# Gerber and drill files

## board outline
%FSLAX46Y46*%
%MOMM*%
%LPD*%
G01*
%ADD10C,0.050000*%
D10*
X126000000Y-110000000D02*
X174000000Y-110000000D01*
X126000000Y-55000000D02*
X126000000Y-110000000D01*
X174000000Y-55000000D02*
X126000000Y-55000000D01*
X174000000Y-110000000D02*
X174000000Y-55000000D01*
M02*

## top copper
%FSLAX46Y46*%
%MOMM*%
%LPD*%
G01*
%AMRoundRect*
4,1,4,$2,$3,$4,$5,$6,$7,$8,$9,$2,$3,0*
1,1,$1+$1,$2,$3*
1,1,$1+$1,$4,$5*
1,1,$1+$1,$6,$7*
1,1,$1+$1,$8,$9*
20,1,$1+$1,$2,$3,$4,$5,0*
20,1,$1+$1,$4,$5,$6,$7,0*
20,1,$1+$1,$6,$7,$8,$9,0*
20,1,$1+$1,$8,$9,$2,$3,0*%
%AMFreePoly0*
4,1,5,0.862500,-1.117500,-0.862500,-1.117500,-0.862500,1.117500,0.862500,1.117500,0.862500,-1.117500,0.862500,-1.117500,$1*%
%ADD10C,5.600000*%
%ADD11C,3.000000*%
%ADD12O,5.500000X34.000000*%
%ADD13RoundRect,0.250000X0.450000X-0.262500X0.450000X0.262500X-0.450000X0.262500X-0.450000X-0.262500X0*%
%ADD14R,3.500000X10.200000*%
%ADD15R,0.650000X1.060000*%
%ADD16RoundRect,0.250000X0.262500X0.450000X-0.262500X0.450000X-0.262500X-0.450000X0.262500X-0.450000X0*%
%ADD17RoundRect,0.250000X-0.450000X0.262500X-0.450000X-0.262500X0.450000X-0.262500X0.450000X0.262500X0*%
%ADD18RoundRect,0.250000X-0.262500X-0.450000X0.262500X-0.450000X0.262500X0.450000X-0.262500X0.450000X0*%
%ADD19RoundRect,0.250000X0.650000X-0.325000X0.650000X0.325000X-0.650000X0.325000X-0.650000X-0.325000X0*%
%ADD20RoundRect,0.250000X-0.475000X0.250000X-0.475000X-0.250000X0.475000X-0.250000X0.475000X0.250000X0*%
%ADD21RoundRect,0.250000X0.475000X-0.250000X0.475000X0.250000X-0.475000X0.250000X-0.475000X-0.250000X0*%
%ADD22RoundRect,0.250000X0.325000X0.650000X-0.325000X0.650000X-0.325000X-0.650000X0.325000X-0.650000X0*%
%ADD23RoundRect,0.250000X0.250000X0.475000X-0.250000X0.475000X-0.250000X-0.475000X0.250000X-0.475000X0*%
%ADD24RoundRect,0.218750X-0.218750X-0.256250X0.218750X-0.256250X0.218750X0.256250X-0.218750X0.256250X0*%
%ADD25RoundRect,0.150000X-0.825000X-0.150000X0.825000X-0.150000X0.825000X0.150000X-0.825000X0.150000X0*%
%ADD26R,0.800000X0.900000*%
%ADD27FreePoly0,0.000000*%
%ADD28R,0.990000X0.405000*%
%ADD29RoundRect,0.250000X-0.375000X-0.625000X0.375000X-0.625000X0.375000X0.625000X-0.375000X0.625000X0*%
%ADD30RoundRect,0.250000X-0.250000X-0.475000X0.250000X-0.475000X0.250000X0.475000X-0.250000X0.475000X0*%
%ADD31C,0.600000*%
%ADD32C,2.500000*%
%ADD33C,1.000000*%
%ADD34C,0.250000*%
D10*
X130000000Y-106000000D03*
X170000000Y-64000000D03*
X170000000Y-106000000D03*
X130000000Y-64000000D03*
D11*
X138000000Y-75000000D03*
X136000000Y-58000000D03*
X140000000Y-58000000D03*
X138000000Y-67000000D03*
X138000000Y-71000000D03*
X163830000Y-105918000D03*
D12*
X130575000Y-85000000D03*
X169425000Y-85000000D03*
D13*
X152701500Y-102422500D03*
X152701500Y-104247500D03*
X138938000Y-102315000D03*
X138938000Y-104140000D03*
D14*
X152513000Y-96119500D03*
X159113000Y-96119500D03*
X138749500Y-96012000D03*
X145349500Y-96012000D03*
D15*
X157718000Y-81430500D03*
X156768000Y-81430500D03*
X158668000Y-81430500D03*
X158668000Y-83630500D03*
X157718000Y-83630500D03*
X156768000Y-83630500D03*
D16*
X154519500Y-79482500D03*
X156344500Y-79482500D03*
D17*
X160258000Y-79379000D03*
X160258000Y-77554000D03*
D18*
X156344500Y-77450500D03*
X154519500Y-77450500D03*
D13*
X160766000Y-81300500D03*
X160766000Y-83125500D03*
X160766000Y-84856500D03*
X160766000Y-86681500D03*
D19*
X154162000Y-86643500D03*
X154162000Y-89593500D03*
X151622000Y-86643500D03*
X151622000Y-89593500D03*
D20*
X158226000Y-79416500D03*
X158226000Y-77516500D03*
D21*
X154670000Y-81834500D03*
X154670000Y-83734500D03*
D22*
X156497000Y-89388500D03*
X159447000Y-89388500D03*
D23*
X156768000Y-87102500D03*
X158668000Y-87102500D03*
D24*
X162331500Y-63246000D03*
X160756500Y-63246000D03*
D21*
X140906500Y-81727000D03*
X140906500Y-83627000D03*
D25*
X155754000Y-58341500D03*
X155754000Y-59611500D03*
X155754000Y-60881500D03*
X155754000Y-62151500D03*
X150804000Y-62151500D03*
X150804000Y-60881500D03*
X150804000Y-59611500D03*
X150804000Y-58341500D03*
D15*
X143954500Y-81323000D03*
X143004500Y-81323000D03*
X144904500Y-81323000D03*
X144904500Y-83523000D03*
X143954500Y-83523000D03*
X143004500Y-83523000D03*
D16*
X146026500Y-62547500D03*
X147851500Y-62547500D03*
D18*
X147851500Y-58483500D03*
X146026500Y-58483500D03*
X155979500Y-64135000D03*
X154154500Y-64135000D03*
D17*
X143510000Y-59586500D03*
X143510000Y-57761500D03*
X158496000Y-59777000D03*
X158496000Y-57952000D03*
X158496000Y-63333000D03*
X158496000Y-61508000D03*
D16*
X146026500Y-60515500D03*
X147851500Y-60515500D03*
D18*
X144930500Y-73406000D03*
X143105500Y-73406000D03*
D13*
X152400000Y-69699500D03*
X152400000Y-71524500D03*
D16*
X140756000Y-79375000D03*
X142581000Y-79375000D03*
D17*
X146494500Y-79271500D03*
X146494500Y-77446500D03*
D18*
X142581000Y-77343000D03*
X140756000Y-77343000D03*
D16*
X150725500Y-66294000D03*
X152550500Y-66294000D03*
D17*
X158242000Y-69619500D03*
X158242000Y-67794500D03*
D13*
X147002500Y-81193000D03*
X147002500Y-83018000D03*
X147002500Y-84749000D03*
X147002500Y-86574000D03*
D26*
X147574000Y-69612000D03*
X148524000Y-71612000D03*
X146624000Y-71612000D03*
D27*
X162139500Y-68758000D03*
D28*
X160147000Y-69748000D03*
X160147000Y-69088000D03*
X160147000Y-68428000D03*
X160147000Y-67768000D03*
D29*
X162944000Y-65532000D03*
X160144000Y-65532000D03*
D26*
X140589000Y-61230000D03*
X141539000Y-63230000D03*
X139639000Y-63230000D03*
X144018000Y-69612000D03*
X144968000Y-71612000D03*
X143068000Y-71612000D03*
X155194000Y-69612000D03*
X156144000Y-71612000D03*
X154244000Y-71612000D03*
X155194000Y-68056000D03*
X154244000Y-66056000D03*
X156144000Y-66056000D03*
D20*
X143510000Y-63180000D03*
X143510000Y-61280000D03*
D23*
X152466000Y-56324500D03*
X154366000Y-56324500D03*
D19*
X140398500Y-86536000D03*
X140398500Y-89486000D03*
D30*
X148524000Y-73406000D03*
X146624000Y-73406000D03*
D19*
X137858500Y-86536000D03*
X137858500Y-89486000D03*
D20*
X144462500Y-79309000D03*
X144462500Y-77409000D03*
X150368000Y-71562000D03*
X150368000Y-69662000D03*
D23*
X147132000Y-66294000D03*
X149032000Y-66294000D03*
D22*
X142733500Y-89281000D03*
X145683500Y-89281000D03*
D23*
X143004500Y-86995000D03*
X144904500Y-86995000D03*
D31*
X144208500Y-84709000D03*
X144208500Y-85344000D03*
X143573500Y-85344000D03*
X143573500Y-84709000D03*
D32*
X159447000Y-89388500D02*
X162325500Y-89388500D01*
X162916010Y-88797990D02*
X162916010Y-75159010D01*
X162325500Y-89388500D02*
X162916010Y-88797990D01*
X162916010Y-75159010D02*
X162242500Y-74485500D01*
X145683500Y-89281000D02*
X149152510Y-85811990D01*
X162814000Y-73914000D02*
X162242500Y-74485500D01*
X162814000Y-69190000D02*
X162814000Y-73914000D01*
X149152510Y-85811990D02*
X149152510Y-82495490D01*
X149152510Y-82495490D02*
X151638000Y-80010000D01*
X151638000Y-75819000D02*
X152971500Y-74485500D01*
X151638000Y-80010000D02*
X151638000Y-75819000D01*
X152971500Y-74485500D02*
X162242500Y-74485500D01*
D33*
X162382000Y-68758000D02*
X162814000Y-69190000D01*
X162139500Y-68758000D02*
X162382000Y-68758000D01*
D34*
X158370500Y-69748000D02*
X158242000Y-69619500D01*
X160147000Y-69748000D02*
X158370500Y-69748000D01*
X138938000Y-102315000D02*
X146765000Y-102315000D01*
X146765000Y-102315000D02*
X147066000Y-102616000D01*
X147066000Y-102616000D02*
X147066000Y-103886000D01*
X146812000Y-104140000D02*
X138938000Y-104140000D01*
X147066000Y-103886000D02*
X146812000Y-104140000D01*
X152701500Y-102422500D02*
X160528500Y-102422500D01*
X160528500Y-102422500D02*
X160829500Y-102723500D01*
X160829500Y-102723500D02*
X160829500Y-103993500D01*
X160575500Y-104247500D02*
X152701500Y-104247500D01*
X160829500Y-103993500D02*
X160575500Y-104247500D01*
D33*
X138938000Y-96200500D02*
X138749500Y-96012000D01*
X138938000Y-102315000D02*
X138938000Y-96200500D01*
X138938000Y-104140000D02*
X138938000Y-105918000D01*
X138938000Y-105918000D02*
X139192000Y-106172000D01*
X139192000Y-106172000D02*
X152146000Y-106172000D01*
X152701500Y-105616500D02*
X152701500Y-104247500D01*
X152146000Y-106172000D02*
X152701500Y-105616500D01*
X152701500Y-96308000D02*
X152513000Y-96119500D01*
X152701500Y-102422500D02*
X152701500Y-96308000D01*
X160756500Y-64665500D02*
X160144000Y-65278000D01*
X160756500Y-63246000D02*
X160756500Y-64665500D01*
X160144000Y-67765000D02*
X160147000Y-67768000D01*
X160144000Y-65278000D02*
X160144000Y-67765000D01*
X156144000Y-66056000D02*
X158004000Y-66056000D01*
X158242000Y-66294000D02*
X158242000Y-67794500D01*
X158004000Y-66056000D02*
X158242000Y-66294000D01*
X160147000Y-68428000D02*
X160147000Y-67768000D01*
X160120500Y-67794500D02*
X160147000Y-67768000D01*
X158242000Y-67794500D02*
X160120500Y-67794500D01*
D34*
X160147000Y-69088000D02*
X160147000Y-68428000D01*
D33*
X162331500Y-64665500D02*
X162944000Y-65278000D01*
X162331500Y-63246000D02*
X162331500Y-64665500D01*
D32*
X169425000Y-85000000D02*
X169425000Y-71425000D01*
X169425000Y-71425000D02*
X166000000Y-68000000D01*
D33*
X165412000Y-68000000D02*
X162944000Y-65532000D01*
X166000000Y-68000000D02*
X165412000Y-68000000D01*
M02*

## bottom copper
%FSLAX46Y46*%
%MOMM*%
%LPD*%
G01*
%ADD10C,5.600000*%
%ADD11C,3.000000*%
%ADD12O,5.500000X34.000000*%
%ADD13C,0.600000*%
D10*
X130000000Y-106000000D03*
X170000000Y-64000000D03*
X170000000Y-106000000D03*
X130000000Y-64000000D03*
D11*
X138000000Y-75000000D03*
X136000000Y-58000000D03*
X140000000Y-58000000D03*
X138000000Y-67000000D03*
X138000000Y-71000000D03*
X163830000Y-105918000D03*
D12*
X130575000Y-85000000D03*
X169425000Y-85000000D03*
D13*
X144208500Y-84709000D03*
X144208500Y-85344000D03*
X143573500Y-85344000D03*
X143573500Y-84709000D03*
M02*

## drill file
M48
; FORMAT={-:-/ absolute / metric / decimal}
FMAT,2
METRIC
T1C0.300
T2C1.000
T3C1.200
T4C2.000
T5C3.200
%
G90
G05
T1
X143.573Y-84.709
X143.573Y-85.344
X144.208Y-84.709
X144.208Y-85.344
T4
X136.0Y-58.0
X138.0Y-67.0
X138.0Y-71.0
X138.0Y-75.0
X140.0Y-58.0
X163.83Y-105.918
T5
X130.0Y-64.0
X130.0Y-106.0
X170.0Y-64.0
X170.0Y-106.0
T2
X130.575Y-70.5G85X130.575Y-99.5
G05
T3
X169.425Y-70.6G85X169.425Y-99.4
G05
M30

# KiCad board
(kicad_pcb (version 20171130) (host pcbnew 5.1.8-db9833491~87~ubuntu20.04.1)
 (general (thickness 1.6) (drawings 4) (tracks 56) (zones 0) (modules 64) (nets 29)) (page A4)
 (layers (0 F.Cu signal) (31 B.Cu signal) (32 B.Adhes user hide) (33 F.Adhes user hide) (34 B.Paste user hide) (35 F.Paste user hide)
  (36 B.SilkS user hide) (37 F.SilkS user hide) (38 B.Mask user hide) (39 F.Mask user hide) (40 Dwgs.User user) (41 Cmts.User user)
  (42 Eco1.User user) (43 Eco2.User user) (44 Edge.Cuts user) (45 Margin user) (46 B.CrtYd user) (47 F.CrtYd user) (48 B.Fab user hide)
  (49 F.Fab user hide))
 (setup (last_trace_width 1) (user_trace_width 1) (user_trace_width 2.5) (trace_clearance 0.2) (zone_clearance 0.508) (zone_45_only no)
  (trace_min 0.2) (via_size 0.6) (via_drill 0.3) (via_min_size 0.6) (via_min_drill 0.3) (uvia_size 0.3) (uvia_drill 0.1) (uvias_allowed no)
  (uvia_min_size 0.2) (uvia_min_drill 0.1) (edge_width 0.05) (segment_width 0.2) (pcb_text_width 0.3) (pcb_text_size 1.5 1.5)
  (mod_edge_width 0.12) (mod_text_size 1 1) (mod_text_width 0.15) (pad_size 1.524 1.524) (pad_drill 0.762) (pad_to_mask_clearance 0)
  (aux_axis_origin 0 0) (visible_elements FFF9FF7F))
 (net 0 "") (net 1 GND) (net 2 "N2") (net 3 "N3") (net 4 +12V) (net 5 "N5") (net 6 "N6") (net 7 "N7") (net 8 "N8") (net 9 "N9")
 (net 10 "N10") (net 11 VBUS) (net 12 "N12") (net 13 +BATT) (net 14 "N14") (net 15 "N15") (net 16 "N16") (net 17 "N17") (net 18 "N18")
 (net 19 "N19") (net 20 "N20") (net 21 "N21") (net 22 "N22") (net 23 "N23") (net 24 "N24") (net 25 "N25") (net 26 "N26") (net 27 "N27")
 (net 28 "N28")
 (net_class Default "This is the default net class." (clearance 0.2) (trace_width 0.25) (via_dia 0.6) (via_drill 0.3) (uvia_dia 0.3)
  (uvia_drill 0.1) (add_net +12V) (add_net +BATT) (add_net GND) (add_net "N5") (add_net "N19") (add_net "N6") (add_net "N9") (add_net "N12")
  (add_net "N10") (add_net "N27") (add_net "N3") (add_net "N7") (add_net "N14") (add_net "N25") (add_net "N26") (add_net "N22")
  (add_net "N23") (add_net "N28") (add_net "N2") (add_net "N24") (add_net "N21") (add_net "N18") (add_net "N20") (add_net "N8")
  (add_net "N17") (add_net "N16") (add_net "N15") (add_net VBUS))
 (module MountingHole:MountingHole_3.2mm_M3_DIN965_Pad (layer F.Cu) (at 130 106)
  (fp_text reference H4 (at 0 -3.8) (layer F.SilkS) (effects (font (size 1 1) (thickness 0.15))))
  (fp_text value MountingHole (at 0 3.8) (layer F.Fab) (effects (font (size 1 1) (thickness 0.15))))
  (pad 1 thru_hole circle (at 0 0) (size 5.6 5.6) (drill 3.2) (layers *.Cu *.Mask)))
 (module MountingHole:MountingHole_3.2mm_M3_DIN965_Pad (layer F.Cu) (at 170 64)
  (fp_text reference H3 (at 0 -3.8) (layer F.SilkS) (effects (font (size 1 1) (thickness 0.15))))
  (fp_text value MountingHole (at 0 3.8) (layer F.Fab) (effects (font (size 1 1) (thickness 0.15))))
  (pad 1 thru_hole circle (at 0 0) (size 5.6 5.6) (drill 3.2) (layers *.Cu *.Mask)))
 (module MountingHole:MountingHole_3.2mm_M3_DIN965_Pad (layer F.Cu) (at 170 106)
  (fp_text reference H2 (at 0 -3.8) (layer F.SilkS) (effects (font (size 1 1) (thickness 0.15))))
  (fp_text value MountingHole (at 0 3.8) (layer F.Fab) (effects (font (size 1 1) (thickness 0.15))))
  (pad 1 thru_hole circle (at 0 0) (size 5.6 5.6) (drill 3.2) (layers *.Cu *.Mask)))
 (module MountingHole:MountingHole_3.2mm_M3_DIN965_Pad (layer F.Cu) (at 130 64)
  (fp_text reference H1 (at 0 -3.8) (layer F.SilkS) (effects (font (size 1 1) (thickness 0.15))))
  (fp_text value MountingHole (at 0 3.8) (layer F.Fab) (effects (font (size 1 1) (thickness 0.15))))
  (pad 1 thru_hole circle (at 0 0) (size 5.6 5.6) (drill 3.2) (layers *.Cu *.Mask)))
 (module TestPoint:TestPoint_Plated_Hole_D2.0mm (layer F.Cu) (at 138 75)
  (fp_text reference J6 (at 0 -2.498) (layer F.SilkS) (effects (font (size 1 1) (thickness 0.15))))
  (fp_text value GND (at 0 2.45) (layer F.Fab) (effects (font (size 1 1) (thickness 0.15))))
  (pad 1 thru_hole circle (at 0 0) (size 3 3) (drill 2) (layers *.Cu *.Mask) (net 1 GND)))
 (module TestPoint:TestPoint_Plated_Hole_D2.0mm (layer F.Cu) (at 136 58)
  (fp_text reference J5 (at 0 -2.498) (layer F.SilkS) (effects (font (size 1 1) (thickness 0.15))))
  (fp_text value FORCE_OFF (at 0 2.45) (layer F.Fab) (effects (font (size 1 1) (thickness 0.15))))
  (pad 1 thru_hole circle (at 0 0) (size 3 3) (drill 2) (layers *.Cu *.Mask) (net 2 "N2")))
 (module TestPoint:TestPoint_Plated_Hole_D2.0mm (layer F.Cu) (at 140 58)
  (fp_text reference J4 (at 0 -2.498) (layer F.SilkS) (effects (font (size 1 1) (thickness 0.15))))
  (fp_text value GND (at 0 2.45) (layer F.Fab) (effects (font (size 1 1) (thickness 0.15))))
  (pad 1 thru_hole circle (at 0 0) (size 3 3) (drill 2) (layers *.Cu *.Mask) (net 1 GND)))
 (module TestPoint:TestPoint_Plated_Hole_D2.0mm (layer F.Cu) (at 138 67)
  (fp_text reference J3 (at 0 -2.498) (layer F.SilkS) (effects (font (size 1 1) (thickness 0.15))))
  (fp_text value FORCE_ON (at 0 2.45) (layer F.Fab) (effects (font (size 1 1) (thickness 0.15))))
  (pad 1 thru_hole circle (at 0 0) (size 3 3) (drill 2) (layers *.Cu *.Mask) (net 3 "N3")))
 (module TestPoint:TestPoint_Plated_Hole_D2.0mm (layer F.Cu) (at 138 71)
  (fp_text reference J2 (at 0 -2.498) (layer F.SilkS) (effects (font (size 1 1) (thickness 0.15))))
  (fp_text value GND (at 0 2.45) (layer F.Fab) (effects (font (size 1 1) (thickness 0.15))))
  (pad 1 thru_hole circle (at 0 0) (size 3 3) (drill 2) (layers *.Cu *.Mask) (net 1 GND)))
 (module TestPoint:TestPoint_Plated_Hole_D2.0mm (layer F.Cu) (at 163.83 105.918)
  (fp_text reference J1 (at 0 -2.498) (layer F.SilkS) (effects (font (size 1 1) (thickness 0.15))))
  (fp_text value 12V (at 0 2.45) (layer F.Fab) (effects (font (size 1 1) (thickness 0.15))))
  (pad 1 thru_hole circle (at 0 0) (size 3 3) (drill 2) (layers *.Cu *.Mask) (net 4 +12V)))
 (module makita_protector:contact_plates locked (layer F.Cu) (at 150 85)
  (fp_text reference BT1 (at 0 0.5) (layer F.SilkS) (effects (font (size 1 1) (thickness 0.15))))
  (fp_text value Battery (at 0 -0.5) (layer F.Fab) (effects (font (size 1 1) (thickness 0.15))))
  (pad 2 thru_hole oval (at -19.425 0) (size 5.5 34) (drill oval 1 30) (layers *.Cu *.Mask) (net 1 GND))
  (pad 1 thru_hole oval (at 19.425 0) (size 5.5 34) (drill oval 1.2 30) (layers *.Cu *.Mask) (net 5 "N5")))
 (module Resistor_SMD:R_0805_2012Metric (layer F.Cu) (at 152.7015 103.335 90)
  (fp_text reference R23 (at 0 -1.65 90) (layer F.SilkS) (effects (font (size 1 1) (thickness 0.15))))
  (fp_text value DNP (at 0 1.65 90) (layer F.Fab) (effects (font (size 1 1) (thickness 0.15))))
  (pad 2 smd roundrect (at 0.9125 0 90) (size 1.025 1.4) (layers F.Cu F.Paste F.Mask) (roundrect_rratio 0.243902) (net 4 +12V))
  (pad 1 smd roundrect (at -0.9125 0 90) (size 1.025 1.4) (layers F.Cu F.Paste F.Mask) (roundrect_rratio 0.243902) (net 4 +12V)))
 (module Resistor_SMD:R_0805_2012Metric (layer F.Cu) (at 138.938 103.2275 90)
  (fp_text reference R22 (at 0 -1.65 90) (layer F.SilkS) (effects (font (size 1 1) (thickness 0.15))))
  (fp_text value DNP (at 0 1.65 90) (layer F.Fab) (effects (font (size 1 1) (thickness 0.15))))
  (pad 2 smd roundrect (at 0.9125 0 90) (size 1.025 1.4) (layers F.Cu F.Paste F.Mask) (roundrect_rratio 0.243902) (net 4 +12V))
  (pad 1 smd roundrect (at -0.9125 0 90) (size 1.025 1.4) (layers F.Cu F.Paste F.Mask) (roundrect_rratio 0.243902) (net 4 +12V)))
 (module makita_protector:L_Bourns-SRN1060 (layer F.Cu) (at 155.813 96.1195 180)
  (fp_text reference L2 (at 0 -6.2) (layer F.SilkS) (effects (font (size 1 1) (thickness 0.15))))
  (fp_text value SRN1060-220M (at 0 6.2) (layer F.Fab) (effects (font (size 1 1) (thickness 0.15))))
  (pad 2 smd rect (at 3.3 0 180) (size 3.5 10.2) (layers F.Cu F.Paste F.Mask) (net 4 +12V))
  (pad 1 smd rect (at -3.3 0 180) (size 3.5 10.2) (layers F.Cu F.Paste F.Mask) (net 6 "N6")))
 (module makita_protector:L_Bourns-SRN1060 (layer F.Cu) (at 142.0495 96.012 180)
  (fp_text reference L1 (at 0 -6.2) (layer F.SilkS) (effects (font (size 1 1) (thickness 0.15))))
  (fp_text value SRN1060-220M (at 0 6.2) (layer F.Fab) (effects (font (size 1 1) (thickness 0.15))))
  (pad 2 smd rect (at 3.3 0 180) (size 3.5 10.2) (layers F.Cu F.Paste F.Mask) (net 4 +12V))
  (pad 1 smd rect (at -3.3 0 180) (size 3.5 10.2) (layers F.Cu F.Paste F.Mask) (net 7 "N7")))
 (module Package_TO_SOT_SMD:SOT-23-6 (layer F.Cu) (at 157.718 82.5305 90)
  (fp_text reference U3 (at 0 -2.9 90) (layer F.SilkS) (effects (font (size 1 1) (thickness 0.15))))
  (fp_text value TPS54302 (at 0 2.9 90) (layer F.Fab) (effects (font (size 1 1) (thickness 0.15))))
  (pad 5 smd rect (at 1.1 0 90) (size 1.06 0.65) (layers F.Cu F.Paste F.Mask) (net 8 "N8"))
  (pad 6 smd rect (at 1.1 -0.95 90) (size 1.06 0.65) (layers F.Cu F.Paste F.Mask) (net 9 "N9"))
  (pad 4 smd rect (at 1.1 0.95 90) (size 1.06 0.65) (layers F.Cu F.Paste F.Mask) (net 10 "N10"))
  (pad 3 smd rect (at -1.1 0.95 90) (size 1.06 0.65) (layers F.Cu F.Paste F.Mask) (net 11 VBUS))
  (pad 2 smd rect (at -1.1 0 90) (size 1.06 0.65) (layers F.Cu F.Paste F.Mask) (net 6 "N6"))
  (pad 1 smd rect (at -1.1 -0.95 90) (size 1.06 0.65) (layers F.Cu F.Paste F.Mask) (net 1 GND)))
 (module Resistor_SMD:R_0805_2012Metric (layer F.Cu) (at 155.432 79.4825 180)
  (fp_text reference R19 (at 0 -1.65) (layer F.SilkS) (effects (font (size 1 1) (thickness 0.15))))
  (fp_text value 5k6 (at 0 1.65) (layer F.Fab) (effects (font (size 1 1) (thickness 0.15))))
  (pad 2 smd roundrect (at 0.9125 0 180) (size 1.025 1.4) (layers F.Cu F.Paste F.Mask) (roundrect_rratio 0.243902) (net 1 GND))
  (pad 1 smd roundrect (at -0.9125 0 180) (size 1.025 1.4) (layers F.Cu F.Paste F.Mask) (roundrect_rratio 0.243902) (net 10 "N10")))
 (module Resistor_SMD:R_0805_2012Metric (layer F.Cu) (at 160.258 78.4665 270)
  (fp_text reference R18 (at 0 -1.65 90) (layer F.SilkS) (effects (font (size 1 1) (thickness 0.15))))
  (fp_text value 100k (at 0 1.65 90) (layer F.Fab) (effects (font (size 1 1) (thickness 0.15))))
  (pad 2 smd roundrect (at 0.9125 0 270) (size 1.025 1.4) (layers F.Cu F.Paste F.Mask) (roundrect_rratio 0.243902) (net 10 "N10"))
  (pad 1 smd roundrect (at -0.9125 0 270) (size 1.025 1.4) (layers F.Cu F.Paste F.Mask) (roundrect_rratio 0.243902) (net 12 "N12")))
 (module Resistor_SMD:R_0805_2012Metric (layer F.Cu) (at 155.432 77.4505)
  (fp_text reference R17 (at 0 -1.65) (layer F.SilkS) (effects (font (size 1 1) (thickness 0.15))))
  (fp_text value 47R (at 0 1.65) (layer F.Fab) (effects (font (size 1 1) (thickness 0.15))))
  (pad 2 smd roundrect (at 0.9125 0) (size 1.025 1.4) (layers F.Cu F.Paste F.Mask) (roundrect_rratio 0.243902) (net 12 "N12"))
  (pad 1 smd roundrect (at -0.9125 0) (size 1.025 1.4) (layers F.Cu F.Paste F.Mask) (roundrect_rratio 0.243902) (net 4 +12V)))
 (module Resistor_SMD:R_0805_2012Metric (layer F.Cu) (at 160.766 82.213 90)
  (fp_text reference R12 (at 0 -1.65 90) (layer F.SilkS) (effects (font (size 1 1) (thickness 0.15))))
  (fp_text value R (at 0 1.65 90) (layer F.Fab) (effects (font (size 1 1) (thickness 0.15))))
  (pad 2 smd roundrect (at 0.9125 0 90) (size 1.025 1.4) (layers F.Cu F.Paste F.Mask) (roundrect_rratio 0.243902) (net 1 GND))
  (pad 1 smd roundrect (at -0.9125 0 90) (size 1.025 1.4) (layers F.Cu F.Paste F.Mask) (roundrect_rratio 0.243902) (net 8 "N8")))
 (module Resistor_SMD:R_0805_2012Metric (layer F.Cu) (at 160.766 85.769 90)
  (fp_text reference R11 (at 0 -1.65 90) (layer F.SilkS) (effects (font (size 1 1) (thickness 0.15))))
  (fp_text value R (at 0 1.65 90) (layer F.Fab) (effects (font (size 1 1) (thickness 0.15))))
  (pad 2 smd roundrect (at 0.9125 0 90) (size 1.025 1.4) (layers F.Cu F.Paste F.Mask) (roundrect_rratio 0.243902) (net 8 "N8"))
  (pad 1 smd roundrect (at -0.9125 0 90) (size 1.025 1.4) (layers F.Cu F.Paste F.Mask) (roundrect_rratio 0.243902) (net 11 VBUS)))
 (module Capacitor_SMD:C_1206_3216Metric (layer F.Cu) (at 154.162 88.1185 90)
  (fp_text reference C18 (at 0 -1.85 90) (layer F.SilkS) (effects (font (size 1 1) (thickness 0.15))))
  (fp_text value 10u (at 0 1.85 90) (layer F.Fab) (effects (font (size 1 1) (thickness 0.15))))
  (pad 2 smd roundrect (at 1.475 0 90) (size 1.15 1.8) (layers F.Cu F.Paste F.Mask) (roundrect_rratio 0.217391) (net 1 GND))
  (pad 1 smd roundrect (at -1.475 0 90) (size 1.15 1.8) (layers F.Cu F.Paste F.Mask) (roundrect_rratio 0.217391) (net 4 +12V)))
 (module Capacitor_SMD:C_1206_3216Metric (layer F.Cu) (at 151.622 88.1185 90)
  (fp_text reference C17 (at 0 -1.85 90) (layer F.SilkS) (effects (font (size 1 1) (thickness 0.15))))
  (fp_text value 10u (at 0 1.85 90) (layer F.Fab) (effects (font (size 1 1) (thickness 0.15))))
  (pad 2 smd roundrect (at 1.475 0 90) (size 1.15 1.8) (layers F.Cu F.Paste F.Mask) (roundrect_rratio 0.217391) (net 1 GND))
  (pad 1 smd roundrect (at -1.475 0 90) (size 1.15 1.8) (layers F.Cu F.Paste F.Mask) (roundrect_rratio 0.217391) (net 4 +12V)))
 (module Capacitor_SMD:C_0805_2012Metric (layer F.Cu) (at 158.226 78.4665 270)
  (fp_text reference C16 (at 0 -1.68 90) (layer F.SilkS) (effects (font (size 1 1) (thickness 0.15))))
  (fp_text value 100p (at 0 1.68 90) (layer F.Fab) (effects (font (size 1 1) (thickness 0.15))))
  (pad 2 smd roundrect (at 0.95 0 270) (size 1 1.45) (layers F.Cu F.Paste F.Mask) (roundrect_rratio 0.25) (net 10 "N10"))
  (pad 1 smd roundrect (at -0.95 0 270) (size 1 1.45) (layers F.Cu F.Paste F.Mask) (roundrect_rratio 0.25) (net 12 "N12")))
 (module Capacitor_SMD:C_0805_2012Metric (layer F.Cu) (at 154.67 82.7845 90)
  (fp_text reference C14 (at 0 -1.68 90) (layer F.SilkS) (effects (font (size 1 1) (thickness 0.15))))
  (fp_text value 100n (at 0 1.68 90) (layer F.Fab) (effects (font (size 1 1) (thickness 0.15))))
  (pad 2 smd roundrect (at 0.95 0 90) (size 1 1.45) (layers F.Cu F.Paste F.Mask) (roundrect_rratio 0.25) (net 9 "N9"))
  (pad 1 smd roundrect (at -0.95 0 90) (size 1 1.45) (layers F.Cu F.Paste F.Mask) (roundrect_rratio 0.25) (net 6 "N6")))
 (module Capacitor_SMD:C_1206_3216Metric (layer F.Cu) (at 157.972 89.3885 180)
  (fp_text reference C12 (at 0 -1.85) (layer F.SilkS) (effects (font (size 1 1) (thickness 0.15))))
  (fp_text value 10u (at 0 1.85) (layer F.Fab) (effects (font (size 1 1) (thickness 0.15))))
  (pad 2 smd roundrect (at 1.475 0 180) (size 1.15 1.8) (layers F.Cu F.Paste F.Mask) (roundrect_rratio 0.217391) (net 1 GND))
  (pad 1 smd roundrect (at -1.475 0 180) (size 1.15 1.8) (layers F.Cu F.Paste F.Mask) (roundrect_rratio 0.217391) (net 11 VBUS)))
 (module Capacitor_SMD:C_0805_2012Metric (layer F.Cu) (at 157.718 87.1025 180)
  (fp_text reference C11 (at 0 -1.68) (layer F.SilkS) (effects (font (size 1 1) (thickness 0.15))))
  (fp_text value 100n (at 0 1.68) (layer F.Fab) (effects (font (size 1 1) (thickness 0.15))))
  (pad 2 smd roundrect (at 0.95 0 180) (size 1 1.45) (layers F.Cu F.Paste F.Mask) (roundrect_rratio 0.25) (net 1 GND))
  (pad 1 smd roundrect (at -0.95 0 180) (size 1 1.45) (layers F.Cu F.Paste F.Mask) (roundrect_rratio 0.25) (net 11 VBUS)))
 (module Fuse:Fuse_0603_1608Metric (layer F.Cu) (at 161.544 63.246)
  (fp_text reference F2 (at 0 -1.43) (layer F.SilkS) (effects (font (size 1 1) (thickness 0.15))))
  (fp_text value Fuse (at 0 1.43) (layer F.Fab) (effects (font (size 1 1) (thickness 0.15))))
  (pad 2 smd roundrect (at 0.7875 0) (size 0.875 0.95) (layers F.Cu F.Paste F.Mask) (roundrect_rratio 0.25) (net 5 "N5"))
  (pad 1 smd roundrect (at -0.7875 0) (size 0.875 0.95) (layers F.Cu F.Paste F.Mask) (roundrect_rratio 0.25) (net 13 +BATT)))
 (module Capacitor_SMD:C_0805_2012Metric (layer F.Cu) (at 140.9065 82.677 90)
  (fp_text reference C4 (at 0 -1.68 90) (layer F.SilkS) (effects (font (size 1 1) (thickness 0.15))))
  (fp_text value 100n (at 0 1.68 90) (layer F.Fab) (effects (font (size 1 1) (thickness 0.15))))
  (pad 2 smd roundrect (at 0.95 0 90) (size 1 1.45) (layers F.Cu F.Paste F.Mask) (roundrect_rratio 0.25) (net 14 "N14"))
  (pad 1 smd roundrect (at -0.95 0 90) (size 1 1.45) (layers F.Cu F.Paste F.Mask) (roundrect_rratio 0.25) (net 7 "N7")))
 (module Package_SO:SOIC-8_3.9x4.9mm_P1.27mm (layer F.Cu) (at 153.279 60.2465)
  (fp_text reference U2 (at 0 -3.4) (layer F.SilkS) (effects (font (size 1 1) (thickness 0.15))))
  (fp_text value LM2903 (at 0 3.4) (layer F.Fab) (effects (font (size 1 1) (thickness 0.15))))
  (pad 8 smd roundrect (at 2.475 -1.905) (size 1.95 0.6) (layers F.Cu F.Paste F.Mask) (roundrect_rratio 0.25) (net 11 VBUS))
  (pad 7 smd roundrect (at 2.475 -0.635) (size 1.95 0.6) (layers F.Cu F.Paste F.Mask) (roundrect_rratio 0.25) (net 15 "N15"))
  (pad 6 smd roundrect (at 2.475 0.635) (size 1.95 0.6) (layers F.Cu F.Paste F.Mask) (roundrect_rratio 0.25) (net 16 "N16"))
  (pad 5 smd roundrect (at 2.475 1.905) (size 1.95 0.6) (layers F.Cu F.Paste F.Mask) (roundrect_rratio 0.25) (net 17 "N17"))
  (pad 4 smd roundrect (at -2.475 1.905) (size 1.95 0.6) (layers F.Cu F.Paste F.Mask) (roundrect_rratio 0.25) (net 1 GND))
  (pad 3 smd roundrect (at -2.475 0.635) (size 1.95 0.6) (layers F.Cu F.Paste F.Mask) (roundrect_rratio 0.25) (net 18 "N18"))
  (pad 2 smd roundrect (at -2.475 -0.635) (size 1.95 0.6) (layers F.Cu F.Paste F.Mask) (roundrect_rratio 0.25) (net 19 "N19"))
  (pad 1 smd roundrect (at -2.475 -1.905) (size 1.95 0.6) (layers F.Cu F.Paste F.Mask) (roundrect_rratio 0.25) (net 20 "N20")))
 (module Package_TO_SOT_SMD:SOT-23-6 (layer F.Cu) (at 143.9545 82.423 90)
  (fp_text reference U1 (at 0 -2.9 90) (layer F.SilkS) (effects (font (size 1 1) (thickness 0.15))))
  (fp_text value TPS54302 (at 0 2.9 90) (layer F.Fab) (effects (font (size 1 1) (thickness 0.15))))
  (pad 5 smd rect (at 1.1 0 90) (size 1.06 0.65) (layers F.Cu F.Paste F.Mask) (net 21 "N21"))
  (pad 6 smd rect (at 1.1 -0.95 90) (size 1.06 0.65) (layers F.Cu F.Paste F.Mask) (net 14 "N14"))
  (pad 4 smd rect (at 1.1 0.95 90) (size 1.06 0.65) (layers F.Cu F.Paste F.Mask) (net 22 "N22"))
  (pad 3 smd rect (at -1.1 0.95 90) (size 1.06 0.65) (layers F.Cu F.Paste F.Mask) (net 11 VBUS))
  (pad 2 smd rect (at -1.1 0 90) (size 1.06 0.65) (layers F.Cu F.Paste F.Mask) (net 7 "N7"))
  (pad 1 smd rect (at -1.1 -0.95 90) (size 1.06 0.65) (layers F.Cu F.Paste F.Mask) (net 1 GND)))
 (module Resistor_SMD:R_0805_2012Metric (layer F.Cu) (at 146.939 62.5475 180)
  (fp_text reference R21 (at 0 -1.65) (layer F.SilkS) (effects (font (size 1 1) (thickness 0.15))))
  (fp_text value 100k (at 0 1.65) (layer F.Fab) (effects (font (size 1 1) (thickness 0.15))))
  (pad 2 smd roundrect (at 0.9125 0 180) (size 1.025 1.4) (layers F.Cu F.Paste F.Mask) (roundrect_rratio 0.243902) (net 1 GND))
  (pad 1 smd roundrect (at -0.9125 0 180) (size 1.025 1.4) (layers F.Cu F.Paste F.Mask) (roundrect_rratio 0.243902) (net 18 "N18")))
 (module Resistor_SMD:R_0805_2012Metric (layer F.Cu) (at 146.939 58.4835)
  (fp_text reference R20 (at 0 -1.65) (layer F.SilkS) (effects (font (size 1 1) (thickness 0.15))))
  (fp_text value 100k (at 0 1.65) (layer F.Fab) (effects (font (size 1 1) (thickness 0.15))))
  (pad 2 smd roundrect (at 0.9125 0) (size 1.025 1.4) (layers F.Cu F.Paste F.Mask) (roundrect_rratio 0.243902) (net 18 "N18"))
  (pad 1 smd roundrect (at -0.9125 0) (size 1.025 1.4) (layers F.Cu F.Paste F.Mask) (roundrect_rratio 0.243902) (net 11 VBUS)))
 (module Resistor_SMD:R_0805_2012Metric (layer F.Cu) (at 155.067 64.135)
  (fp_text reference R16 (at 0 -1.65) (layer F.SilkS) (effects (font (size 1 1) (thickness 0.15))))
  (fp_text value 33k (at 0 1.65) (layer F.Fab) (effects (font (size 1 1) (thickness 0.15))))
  (pad 2 smd roundrect (at 0.9125 0) (size 1.025 1.4) (layers F.Cu F.Paste F.Mask) (roundrect_rratio 0.243902) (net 2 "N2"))
  (pad 1 smd roundrect (at -0.9125 0) (size 1.025 1.4) (layers F.Cu F.Paste F.Mask) (roundrect_rratio 0.243902) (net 18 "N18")))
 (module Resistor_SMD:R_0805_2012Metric (layer F.Cu) (at 143.51 58.674 270)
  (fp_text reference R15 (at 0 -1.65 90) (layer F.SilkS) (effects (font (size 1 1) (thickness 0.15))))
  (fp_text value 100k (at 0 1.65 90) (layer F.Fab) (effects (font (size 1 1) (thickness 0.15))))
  (pad 2 smd roundrect (at 0.9125 0 270) (size 1.025 1.4) (layers F.Cu F.Paste F.Mask) (roundrect_rratio 0.243902) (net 19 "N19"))
  (pad 1 smd roundrect (at -0.9125 0 270) (size 1.025 1.4) (layers F.Cu F.Paste F.Mask) (roundrect_rratio 0.243902) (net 11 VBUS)))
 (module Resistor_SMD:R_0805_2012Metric (layer F.Cu) (at 158.496 58.8645 270)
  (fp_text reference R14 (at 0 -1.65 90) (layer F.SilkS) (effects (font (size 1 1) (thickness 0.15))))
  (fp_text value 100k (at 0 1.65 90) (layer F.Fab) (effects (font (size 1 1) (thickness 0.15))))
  (pad 2 smd roundrect (at 0.9125 0 270) (size 1.025 1.4) (layers F.Cu F.Paste F.Mask) (roundrect_rratio 0.243902) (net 16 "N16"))
  (pad 1 smd roundrect (at -0.9125 0 270) (size 1.025 1.4) (layers F.Cu F.Paste F.Mask) (roundrect_rratio 0.243902) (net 11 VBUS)))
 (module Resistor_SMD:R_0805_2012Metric (layer F.Cu) (at 158.496 62.4205 270)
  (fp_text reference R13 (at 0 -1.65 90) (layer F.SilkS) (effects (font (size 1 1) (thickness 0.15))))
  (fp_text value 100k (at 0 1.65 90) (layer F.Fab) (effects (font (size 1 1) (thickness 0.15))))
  (pad 2 smd roundrect (at 0.9125 0 270) (size 1.025 1.4) (layers F.Cu F.Paste F.Mask) (roundrect_rratio 0.243902) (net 1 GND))
  (pad 1 smd roundrect (at -0.9125 0 270) (size 1.025 1.4) (layers F.Cu F.Paste F.Mask) (roundrect_rratio 0.243902) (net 17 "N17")))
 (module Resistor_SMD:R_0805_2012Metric (layer F.Cu) (at 146.939 60.5155 180)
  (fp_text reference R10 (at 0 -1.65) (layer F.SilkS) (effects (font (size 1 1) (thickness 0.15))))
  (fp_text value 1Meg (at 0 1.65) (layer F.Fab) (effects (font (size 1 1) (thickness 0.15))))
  (pad 2 smd roundrect (at 0.9125 0 180) (size 1.025 1.4) (layers F.Cu F.Paste F.Mask) (roundrect_rratio 0.243902) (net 20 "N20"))
  (pad 1 smd roundrect (at -0.9125 0 180) (size 1.025 1.4) (layers F.Cu F.Paste F.Mask) (roundrect_rratio 0.243902) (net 18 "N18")))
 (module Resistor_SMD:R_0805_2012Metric (layer F.Cu) (at 144.018 73.406)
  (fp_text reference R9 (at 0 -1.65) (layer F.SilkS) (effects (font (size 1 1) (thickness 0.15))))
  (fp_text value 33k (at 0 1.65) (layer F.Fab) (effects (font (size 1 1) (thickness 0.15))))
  (pad 2 smd roundrect (at 0.9125 0) (size 1.025 1.4) (layers F.Cu F.Paste F.Mask) (roundrect_rratio 0.243902) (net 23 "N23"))
  (pad 1 smd roundrect (at -0.9125 0) (size 1.025 1.4) (layers F.Cu F.Paste F.Mask) (roundrect_rratio 0.243902) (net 20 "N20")))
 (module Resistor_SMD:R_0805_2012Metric (layer F.Cu) (at 152.4 70.612 90)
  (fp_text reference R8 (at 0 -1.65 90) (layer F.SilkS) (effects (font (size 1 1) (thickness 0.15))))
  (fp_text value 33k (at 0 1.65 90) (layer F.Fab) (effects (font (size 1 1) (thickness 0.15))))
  (pad 2 smd roundrect (at 0.9125 0 90) (size 1.025 1.4) (layers F.Cu F.Paste F.Mask) (roundrect_rratio 0.243902) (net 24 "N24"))
  (pad 1 smd roundrect (at -0.9125 0 90) (size 1.025 1.4) (layers F.Cu F.Paste F.Mask) (roundrect_rratio 0.243902) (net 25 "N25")))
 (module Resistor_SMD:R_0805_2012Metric (layer F.Cu) (at 141.6685 79.375 180)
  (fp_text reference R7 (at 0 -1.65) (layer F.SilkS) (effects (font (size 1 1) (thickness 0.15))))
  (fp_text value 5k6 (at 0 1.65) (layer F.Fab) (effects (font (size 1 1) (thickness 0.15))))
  (pad 2 smd roundrect (at 0.9125 0 180) (size 1.025 1.4) (layers F.Cu F.Paste F.Mask) (roundrect_rratio 0.243902) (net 1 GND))
  (pad 1 smd roundrect (at -0.9125 0 180) (size 1.025 1.4) (layers F.Cu F.Paste F.Mask) (roundrect_rratio 0.243902) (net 22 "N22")))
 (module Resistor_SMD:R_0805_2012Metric (layer F.Cu) (at 146.4945 78.359 270)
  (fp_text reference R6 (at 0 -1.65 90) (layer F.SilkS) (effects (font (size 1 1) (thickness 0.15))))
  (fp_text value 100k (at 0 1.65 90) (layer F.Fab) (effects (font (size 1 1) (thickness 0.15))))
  (pad 2 smd roundrect (at 0.9125 0 270) (size 1.025 1.4) (layers F.Cu F.Paste F.Mask) (roundrect_rratio 0.243902) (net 22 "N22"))
  (pad 1 smd roundrect (at -0.9125 0 270) (size 1.025 1.4) (layers F.Cu F.Paste F.Mask) (roundrect_rratio 0.243902) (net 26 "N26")))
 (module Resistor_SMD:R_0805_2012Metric (layer F.Cu) (at 141.6685 77.343)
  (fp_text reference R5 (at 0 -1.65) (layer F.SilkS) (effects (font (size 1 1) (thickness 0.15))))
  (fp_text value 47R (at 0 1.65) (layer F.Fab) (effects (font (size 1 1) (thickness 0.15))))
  (pad 2 smd roundrect (at 0.9125 0) (size 1.025 1.4) (layers F.Cu F.Paste F.Mask) (roundrect_rratio 0.243902) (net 26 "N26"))
  (pad 1 smd roundrect (at -0.9125 0) (size 1.025 1.4) (layers F.Cu F.Paste F.Mask) (roundrect_rratio 0.243902) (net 4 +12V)))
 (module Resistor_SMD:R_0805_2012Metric (layer F.Cu) (at 151.638 66.294 180)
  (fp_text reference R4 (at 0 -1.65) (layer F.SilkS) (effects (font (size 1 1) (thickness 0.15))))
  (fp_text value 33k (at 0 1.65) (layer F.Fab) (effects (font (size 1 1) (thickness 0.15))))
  (pad 2 smd roundrect (at 0.9125 0 180) (size 1.025 1.4) (layers F.Cu F.Paste F.Mask) (roundrect_rratio 0.243902) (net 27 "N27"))
  (pad 1 smd roundrect (at -0.9125 0 180) (size 1.025 1.4) (layers F.Cu F.Paste F.Mask) (roundrect_rratio 0.243902) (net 25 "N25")))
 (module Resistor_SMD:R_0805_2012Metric (layer F.Cu) (at 158.242 68.707 270)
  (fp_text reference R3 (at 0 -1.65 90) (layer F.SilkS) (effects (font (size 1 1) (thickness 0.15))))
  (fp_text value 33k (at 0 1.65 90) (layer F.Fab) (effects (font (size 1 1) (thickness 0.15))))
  (pad 2 smd roundrect (at 0.9125 0 270) (size 1.025 1.4) (layers F.Cu F.Paste F.Mask) (roundrect_rratio 0.243902) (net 25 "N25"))
  (pad 1 smd roundrect (at -0.9125 0 270) (size 1.025 1.4) (layers F.Cu F.Paste F.Mask) (roundrect_rratio 0.243902) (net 13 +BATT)))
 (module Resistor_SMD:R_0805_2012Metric (layer F.Cu) (at 147.0025 82.1055 90)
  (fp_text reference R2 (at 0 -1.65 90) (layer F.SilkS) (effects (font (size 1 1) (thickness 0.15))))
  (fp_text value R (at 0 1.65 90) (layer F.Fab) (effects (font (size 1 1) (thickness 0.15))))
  (pad 2 smd roundrect (at 0.9125 0 90) (size 1.025 1.4) (layers F.Cu F.Paste F.Mask) (roundrect_rratio 0.243902) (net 1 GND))
  (pad 1 smd roundrect (at -0.9125 0 90) (size 1.025 1.4) (layers F.Cu F.Paste F.Mask) (roundrect_rratio 0.243902) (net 21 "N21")))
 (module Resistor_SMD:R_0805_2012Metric (layer F.Cu) (at 147.0025 85.6615 90)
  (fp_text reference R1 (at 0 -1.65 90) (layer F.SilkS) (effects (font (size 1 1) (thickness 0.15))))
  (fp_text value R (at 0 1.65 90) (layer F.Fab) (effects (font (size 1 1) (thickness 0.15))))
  (pad 2 smd roundrect (at 0.9125 0 90) (size 1.025 1.4) (layers F.Cu F.Paste F.Mask) (roundrect_rratio 0.243902) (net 21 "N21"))
  (pad 1 smd roundrect (at -0.9125 0 90) (size 1.025 1.4) (layers F.Cu F.Paste F.Mask) (roundrect_rratio 0.243902) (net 11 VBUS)))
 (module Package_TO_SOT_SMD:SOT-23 (layer F.Cu) (at 147.574 70.612 90)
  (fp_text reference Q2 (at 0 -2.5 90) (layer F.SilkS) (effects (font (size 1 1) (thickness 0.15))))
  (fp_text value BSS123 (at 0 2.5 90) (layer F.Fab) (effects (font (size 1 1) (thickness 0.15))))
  (pad 3 smd rect (at 1 0 90) (size 0.9 0.8) (layers F.Cu F.Paste F.Mask) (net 24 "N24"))
  (pad 2 smd rect (at -1 0.95 90) (size 0.9 0.8) (layers F.Cu F.Paste F.Mask) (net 1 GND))
  (pad 1 smd rect (at -1 -0.95 90) (size 0.9 0.8) (layers F.Cu F.Paste F.Mask) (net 23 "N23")))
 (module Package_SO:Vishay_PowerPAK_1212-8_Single (layer F.Cu) (at 161.582 68.758)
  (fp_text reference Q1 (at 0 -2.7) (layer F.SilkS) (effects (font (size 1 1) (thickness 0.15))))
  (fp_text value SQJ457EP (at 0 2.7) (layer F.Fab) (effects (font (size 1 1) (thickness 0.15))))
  (pad 5 smd custom (at 0.5575 0) (size 1.725 2.235) (layers F.Cu F.Paste F.Mask) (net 11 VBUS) (zone_connect 2)
   (options (clearance outline) (anchor rect)) (primitives))
  (pad 4 smd rect (at -1.435 0.99) (size 0.99 0.405) (layers F.Cu F.Paste F.Mask) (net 25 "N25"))
  (pad 3 smd rect (at -1.435 0.33) (size 0.99 0.405) (layers F.Cu F.Paste F.Mask) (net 13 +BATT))
  (pad 2 smd rect (at -1.435 -0.33) (size 0.99 0.405) (layers F.Cu F.Paste F.Mask) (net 13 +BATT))
  (pad 1 smd rect (at -1.435 -0.99) (size 0.99 0.405) (layers F.Cu F.Paste F.Mask) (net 13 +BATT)))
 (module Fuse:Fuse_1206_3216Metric (layer F.Cu) (at 161.544 65.532)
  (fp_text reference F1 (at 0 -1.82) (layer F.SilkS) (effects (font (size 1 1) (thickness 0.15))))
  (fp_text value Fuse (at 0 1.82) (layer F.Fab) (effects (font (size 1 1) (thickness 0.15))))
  (pad 2 smd roundrect (at 1.4 0) (size 1.25 1.75) (layers F.Cu F.Paste F.Mask) (roundrect_rratio 0.2) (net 5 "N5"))
  (pad 1 smd roundrect (at -1.4 0) (size 1.25 1.75) (layers F.Cu F.Paste F.Mask) (roundrect_rratio 0.2) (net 13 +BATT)))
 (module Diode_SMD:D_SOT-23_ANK (layer F.Cu) (at 140.589 62.23 90)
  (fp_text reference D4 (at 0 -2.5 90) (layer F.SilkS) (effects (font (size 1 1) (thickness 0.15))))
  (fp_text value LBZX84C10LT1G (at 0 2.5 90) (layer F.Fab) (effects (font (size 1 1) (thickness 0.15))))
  (pad 1 smd rect (at 1 0 90) (size 0.9 0.8) (layers F.Cu F.Paste F.Mask) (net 19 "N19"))
  (pad "" smd rect (at -1 0.95 90) (size 0.9 0.8) (layers F.Cu F.Paste F.Mask))
  (pad 2 smd rect (at -1 -0.95 90) (size 0.9 0.8) (layers F.Cu F.Paste F.Mask) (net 1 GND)))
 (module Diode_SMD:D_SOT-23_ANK (layer F.Cu) (at 144.018 70.612 90)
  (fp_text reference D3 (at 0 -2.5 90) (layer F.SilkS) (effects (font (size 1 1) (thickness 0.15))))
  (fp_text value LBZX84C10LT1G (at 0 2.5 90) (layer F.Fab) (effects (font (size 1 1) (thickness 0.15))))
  (pad 1 smd rect (at 1 0 90) (size 0.9 0.8) (layers F.Cu F.Paste F.Mask) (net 23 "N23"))
  (pad "" smd rect (at -1 0.95 90) (size 0.9 0.8) (layers F.Cu F.Paste F.Mask))
  (pad 2 smd rect (at -1 -0.95 90) (size 0.9 0.8) (layers F.Cu F.Paste F.Mask) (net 1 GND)))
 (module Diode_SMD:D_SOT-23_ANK (layer F.Cu) (at 155.194 70.612 90)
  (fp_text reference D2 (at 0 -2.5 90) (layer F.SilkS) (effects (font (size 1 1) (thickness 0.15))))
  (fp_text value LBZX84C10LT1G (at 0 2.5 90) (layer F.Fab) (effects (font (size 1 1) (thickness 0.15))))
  (pad 1 smd rect (at 1 0 90) (size 0.9 0.8) (layers F.Cu F.Paste F.Mask) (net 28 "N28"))
  (pad "" smd rect (at -1 0.95 90) (size 0.9 0.8) (layers F.Cu F.Paste F.Mask))
  (pad 2 smd rect (at -1 -0.95 90) (size 0.9 0.8) (layers F.Cu F.Paste F.Mask) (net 25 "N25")))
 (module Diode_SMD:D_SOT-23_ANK (layer F.Cu) (at 155.194 67.056 270)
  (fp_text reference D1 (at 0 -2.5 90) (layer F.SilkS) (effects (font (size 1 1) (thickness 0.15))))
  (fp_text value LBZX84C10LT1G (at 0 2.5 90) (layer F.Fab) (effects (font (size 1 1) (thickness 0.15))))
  (pad 1 smd rect (at 1 0 270) (size 0.9 0.8) (layers F.Cu F.Paste F.Mask) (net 28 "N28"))
  (pad "" smd rect (at -1 0.95 270) (size 0.9 0.8) (layers F.Cu F.Paste F.Mask))
  (pad 2 smd rect (at -1 -0.95 270) (size 0.9 0.8) (layers F.Cu F.Paste F.Mask) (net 13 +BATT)))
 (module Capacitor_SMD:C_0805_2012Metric (layer F.Cu) (at 143.51 62.23 270)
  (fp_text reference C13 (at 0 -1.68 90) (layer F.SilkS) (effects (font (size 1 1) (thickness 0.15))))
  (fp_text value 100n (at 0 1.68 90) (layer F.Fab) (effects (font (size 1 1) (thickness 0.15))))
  (pad 2 smd roundrect (at 0.95 0 270) (size 1 1.45) (layers F.Cu F.Paste F.Mask) (roundrect_rratio 0.25) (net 1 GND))
  (pad 1 smd roundrect (at -0.95 0 270) (size 1 1.45) (layers F.Cu F.Paste F.Mask) (roundrect_rratio 0.25) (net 19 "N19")))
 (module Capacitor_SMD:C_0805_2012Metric (layer F.Cu) (at 153.416 56.3245 180)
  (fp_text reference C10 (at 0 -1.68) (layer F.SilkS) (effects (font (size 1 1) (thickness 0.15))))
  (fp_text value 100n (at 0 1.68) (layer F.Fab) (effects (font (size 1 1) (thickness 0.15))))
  (pad 2 smd roundrect (at 0.95 0 180) (size 1 1.45) (layers F.Cu F.Paste F.Mask) (roundrect_rratio 0.25) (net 1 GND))
  (pad 1 smd roundrect (at -0.95 0 180) (size 1 1.45) (layers F.Cu F.Paste F.Mask) (roundrect_rratio 0.25) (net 11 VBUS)))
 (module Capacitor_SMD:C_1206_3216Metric (layer F.Cu) (at 140.3985 88.011 90)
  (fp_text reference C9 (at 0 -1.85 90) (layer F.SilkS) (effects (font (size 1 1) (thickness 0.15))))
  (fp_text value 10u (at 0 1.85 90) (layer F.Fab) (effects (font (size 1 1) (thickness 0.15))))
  (pad 2 smd roundrect (at 1.475 0 90) (size 1.15 1.8) (layers F.Cu F.Paste F.Mask) (roundrect_rratio 0.217391) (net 1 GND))
  (pad 1 smd roundrect (at -1.475 0 90) (size 1.15 1.8) (layers F.Cu F.Paste F.Mask) (roundrect_rratio 0.217391) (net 4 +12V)))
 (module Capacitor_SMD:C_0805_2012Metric (layer F.Cu) (at 147.574 73.406)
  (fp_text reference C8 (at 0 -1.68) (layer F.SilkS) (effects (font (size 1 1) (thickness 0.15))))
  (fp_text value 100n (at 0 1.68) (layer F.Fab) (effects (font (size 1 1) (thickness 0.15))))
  (pad 2 smd roundrect (at 0.95 0) (size 1 1.45) (layers F.Cu F.Paste F.Mask) (roundrect_rratio 0.25) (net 1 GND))
  (pad 1 smd roundrect (at -0.95 0) (size 1 1.45) (layers F.Cu F.Paste F.Mask) (roundrect_rratio 0.25) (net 23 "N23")))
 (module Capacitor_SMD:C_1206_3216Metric (layer F.Cu) (at 137.8585 88.011 90)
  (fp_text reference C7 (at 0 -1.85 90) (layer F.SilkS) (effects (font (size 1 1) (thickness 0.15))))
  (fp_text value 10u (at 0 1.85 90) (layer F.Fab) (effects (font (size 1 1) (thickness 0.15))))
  (pad 2 smd roundrect (at 1.475 0 90) (size 1.15 1.8) (layers F.Cu F.Paste F.Mask) (roundrect_rratio 0.217391) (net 1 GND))
  (pad 1 smd roundrect (at -1.475 0 90) (size 1.15 1.8) (layers F.Cu F.Paste F.Mask) (roundrect_rratio 0.217391) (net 4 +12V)))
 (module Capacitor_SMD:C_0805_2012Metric (layer F.Cu) (at 144.4625 78.359 270)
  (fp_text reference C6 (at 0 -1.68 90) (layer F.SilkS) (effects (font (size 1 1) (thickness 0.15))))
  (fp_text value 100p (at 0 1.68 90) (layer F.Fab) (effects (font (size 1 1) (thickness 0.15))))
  (pad 2 smd roundrect (at 0.95 0 270) (size 1 1.45) (layers F.Cu F.Paste F.Mask) (roundrect_rratio 0.25) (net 22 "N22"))
  (pad 1 smd roundrect (at -0.95 0 270) (size 1 1.45) (layers F.Cu F.Paste F.Mask) (roundrect_rratio 0.25) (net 26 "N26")))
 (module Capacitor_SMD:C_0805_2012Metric (layer F.Cu) (at 150.368 70.612 270)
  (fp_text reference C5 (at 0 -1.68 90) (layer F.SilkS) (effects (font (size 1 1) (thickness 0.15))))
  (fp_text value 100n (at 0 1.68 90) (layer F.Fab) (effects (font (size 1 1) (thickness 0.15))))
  (pad 2 smd roundrect (at 0.95 0 270) (size 1 1.45) (layers F.Cu F.Paste F.Mask) (roundrect_rratio 0.25) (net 1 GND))
  (pad 1 smd roundrect (at -0.95 0 270) (size 1 1.45) (layers F.Cu F.Paste F.Mask) (roundrect_rratio 0.25) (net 25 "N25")))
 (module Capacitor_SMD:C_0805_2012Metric (layer F.Cu) (at 148.082 66.294 180)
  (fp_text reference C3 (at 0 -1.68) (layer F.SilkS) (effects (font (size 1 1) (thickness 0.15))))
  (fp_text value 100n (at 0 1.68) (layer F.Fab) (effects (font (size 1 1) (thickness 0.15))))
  (pad 2 smd roundrect (at 0.95 0 180) (size 1 1.45) (layers F.Cu F.Paste F.Mask) (roundrect_rratio 0.25) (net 3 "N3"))
  (pad 1 smd roundrect (at -0.95 0 180) (size 1 1.45) (layers F.Cu F.Paste F.Mask) (roundrect_rratio 0.25) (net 27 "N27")))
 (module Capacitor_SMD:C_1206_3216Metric (layer F.Cu) (at 144.2085 89.281 180)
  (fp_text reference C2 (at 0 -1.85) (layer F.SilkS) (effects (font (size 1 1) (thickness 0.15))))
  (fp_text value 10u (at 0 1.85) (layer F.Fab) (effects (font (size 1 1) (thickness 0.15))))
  (pad 2 smd roundrect (at 1.475 0 180) (size 1.15 1.8) (layers F.Cu F.Paste F.Mask) (roundrect_rratio 0.217391) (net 1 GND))
  (pad 1 smd roundrect (at -1.475 0 180) (size 1.15 1.8) (layers F.Cu F.Paste F.Mask) (roundrect_rratio 0.217391) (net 11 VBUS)))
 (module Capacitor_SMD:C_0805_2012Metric (layer F.Cu) (at 143.9545 86.995 180)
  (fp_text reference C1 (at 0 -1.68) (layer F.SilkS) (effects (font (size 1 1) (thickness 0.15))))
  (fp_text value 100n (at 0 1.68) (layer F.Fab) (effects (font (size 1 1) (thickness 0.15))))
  (pad 2 smd roundrect (at 0.95 0 180) (size 1 1.45) (layers F.Cu F.Paste F.Mask) (roundrect_rratio 0.25) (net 1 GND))
  (pad 1 smd roundrect (at -0.95 0 180) (size 1 1.45) (layers F.Cu F.Paste F.Mask) (roundrect_rratio 0.25) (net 11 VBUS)))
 (gr_line (start 126 110) (end 174 110) (layer Edge.Cuts) (width 0.05))
 (gr_line (start 126 55) (end 126 110) (layer Edge.Cuts) (width 0.05))
 (gr_line (start 174 55) (end 126 55) (layer Edge.Cuts) (width 0.05))
 (gr_line (start 174 110) (end 174 55) (layer Edge.Cuts) (width 0.05))
 (via (at 144.2085 84.709) (size 0.6) (drill 0.3) (layers F.Cu B.Cu) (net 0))
 (via (at 144.2085 85.344) (size 0.6) (drill 0.3) (layers F.Cu B.Cu) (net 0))
 (via (at 143.5735 85.344) (size 0.6) (drill 0.3) (layers F.Cu B.Cu) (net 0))
 (via (at 143.5735 84.709) (size 0.6) (drill 0.3) (layers F.Cu B.Cu) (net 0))
 (segment (start 159.447 89.3885) (end 162.3255 89.3885) (width 2.5) (layer F.Cu) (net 11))
 (segment (start 162.91601 88.79799) (end 162.91601 75.15901) (width 2.5) (layer F.Cu) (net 11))
 (segment (start 162.3255 89.3885) (end 162.91601 88.79799) (width 2.5) (layer F.Cu) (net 11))
 (segment (start 162.91601 75.15901) (end 162.2425 74.4855) (width 2.5) (layer F.Cu) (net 11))
 (segment (start 145.6835 89.281) (end 149.15251 85.81199) (width 2.5) (layer F.Cu) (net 11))
 (segment (start 162.814 73.914) (end 162.2425 74.4855) (width 2.5) (layer F.Cu) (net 11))
 (segment (start 162.814 69.19) (end 162.814 73.914) (width 2.5) (layer F.Cu) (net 11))
 (segment (start 149.15251 85.81199) (end 149.15251 82.49549) (width 2.5) (layer F.Cu) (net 11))
 (segment (start 149.15251 82.49549) (end 151.638 80.01) (width 2.5) (layer F.Cu) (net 11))
 (segment (start 151.638 75.819) (end 152.9715 74.4855) (width 2.5) (layer F.Cu) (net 11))
 (segment (start 151.638 80.01) (end 151.638 75.819) (width 2.5) (layer F.Cu) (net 11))
 (segment (start 152.9715 74.4855) (end 162.2425 74.4855) (width 2.5) (layer F.Cu) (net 11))
 (segment (start 162.382 68.758) (end 162.814 69.19) (width 1) (layer F.Cu) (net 11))
 (segment (start 162.1395 68.758) (end 162.382 68.758) (width 1) (layer F.Cu) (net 11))
 (segment (start 158.3705 69.748) (end 158.242 69.6195) (width 0.25) (layer F.Cu) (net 25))
 (segment (start 160.147 69.748) (end 158.3705 69.748) (width 0.25) (layer F.Cu) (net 25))
 (segment (start 138.938 102.315) (end 146.765 102.315) (width 0.25) (layer F.Cu) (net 4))
 (segment (start 146.765 102.315) (end 147.066 102.616) (width 0.25) (layer F.Cu) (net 4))
 (segment (start 147.066 102.616) (end 147.066 103.886) (width 0.25) (layer F.Cu) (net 4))
 (segment (start 146.812 104.14) (end 138.938 104.14) (width 0.25) (layer F.Cu) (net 4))
 (segment (start 147.066 103.886) (end 146.812 104.14) (width 0.25) (layer F.Cu) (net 4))
 (segment (start 152.7015 102.4225) (end 160.5285 102.4225) (width 0.25) (layer F.Cu) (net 4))
 (segment (start 160.5285 102.4225) (end 160.8295 102.7235) (width 0.25) (layer F.Cu) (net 4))
 (segment (start 160.8295 102.7235) (end 160.8295 103.9935) (width 0.25) (layer F.Cu) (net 4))
 (segment (start 160.5755 104.2475) (end 152.7015 104.2475) (width 0.25) (layer F.Cu) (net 4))
 (segment (start 160.8295 103.9935) (end 160.5755 104.2475) (width 0.25) (layer F.Cu) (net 4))
 (segment (start 138.938 96.2005) (end 138.7495 96.012) (width 1) (layer F.Cu) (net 4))
 (segment (start 138.938 102.315) (end 138.938 96.2005) (width 1) (layer F.Cu) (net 4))
 (segment (start 138.938 104.14) (end 138.938 105.918) (width 1) (layer F.Cu) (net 4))
 (segment (start 138.938 105.918) (end 139.192 106.172) (width 1) (layer F.Cu) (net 4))
 (segment (start 139.192 106.172) (end 152.146 106.172) (width 1) (layer F.Cu) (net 4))
 (segment (start 152.7015 105.6165) (end 152.7015 104.2475) (width 1) (layer F.Cu) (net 4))
 (segment (start 152.146 106.172) (end 152.7015 105.6165) (width 1) (layer F.Cu) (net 4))
 (segment (start 152.7015 96.308) (end 152.513 96.1195) (width 1) (layer F.Cu) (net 4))
 (segment (start 152.7015 102.4225) (end 152.7015 96.308) (width 1) (layer F.Cu) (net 4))
 (segment (start 160.7565 64.6655) (end 160.144 65.278) (width 1) (layer F.Cu) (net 13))
 (segment (start 160.7565 63.246) (end 160.7565 64.6655) (width 1) (layer F.Cu) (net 13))
 (segment (start 160.144 67.765) (end 160.147 67.768) (width 1) (layer F.Cu) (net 13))
 (segment (start 160.144 65.278) (end 160.144 67.765) (width 1) (layer F.Cu) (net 13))
 (segment (start 156.144 66.056) (end 158.004 66.056) (width 1) (layer F.Cu) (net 13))
 (segment (start 158.242 66.294) (end 158.242 67.7945) (width 1) (layer F.Cu) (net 13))
 (segment (start 158.004 66.056) (end 158.242 66.294) (width 1) (layer F.Cu) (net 13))
 (segment (start 160.147 68.428) (end 160.147 67.768) (width 1) (layer F.Cu) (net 13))
 (segment (start 160.1205 67.7945) (end 160.147 67.768) (width 1) (layer F.Cu) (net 13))
 (segment (start 158.242 67.7945) (end 160.1205 67.7945) (width 1) (layer F.Cu) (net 13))
 (segment (start 160.147 69.088) (end 160.147 68.428) (width 0.25) (layer F.Cu) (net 13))
 (segment (start 162.3315 64.6655) (end 162.944 65.278) (width 1) (layer F.Cu) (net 5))
 (segment (start 162.3315 63.246) (end 162.3315 64.6655) (width 1) (layer F.Cu) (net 5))
 (segment (start 169.425 85) (end 169.425 71.425) (width 2.5) (layer F.Cu) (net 5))
 (segment (start 169.425 71.425) (end 166 68) (width 2.5) (layer F.Cu) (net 5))
 (segment (start 165.412 68) (end 162.944 65.532) (width 1) (layer F.Cu) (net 5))
 (segment (start 166 68) (end 165.412 68) (width 1) (layer F.Cu) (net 5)))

